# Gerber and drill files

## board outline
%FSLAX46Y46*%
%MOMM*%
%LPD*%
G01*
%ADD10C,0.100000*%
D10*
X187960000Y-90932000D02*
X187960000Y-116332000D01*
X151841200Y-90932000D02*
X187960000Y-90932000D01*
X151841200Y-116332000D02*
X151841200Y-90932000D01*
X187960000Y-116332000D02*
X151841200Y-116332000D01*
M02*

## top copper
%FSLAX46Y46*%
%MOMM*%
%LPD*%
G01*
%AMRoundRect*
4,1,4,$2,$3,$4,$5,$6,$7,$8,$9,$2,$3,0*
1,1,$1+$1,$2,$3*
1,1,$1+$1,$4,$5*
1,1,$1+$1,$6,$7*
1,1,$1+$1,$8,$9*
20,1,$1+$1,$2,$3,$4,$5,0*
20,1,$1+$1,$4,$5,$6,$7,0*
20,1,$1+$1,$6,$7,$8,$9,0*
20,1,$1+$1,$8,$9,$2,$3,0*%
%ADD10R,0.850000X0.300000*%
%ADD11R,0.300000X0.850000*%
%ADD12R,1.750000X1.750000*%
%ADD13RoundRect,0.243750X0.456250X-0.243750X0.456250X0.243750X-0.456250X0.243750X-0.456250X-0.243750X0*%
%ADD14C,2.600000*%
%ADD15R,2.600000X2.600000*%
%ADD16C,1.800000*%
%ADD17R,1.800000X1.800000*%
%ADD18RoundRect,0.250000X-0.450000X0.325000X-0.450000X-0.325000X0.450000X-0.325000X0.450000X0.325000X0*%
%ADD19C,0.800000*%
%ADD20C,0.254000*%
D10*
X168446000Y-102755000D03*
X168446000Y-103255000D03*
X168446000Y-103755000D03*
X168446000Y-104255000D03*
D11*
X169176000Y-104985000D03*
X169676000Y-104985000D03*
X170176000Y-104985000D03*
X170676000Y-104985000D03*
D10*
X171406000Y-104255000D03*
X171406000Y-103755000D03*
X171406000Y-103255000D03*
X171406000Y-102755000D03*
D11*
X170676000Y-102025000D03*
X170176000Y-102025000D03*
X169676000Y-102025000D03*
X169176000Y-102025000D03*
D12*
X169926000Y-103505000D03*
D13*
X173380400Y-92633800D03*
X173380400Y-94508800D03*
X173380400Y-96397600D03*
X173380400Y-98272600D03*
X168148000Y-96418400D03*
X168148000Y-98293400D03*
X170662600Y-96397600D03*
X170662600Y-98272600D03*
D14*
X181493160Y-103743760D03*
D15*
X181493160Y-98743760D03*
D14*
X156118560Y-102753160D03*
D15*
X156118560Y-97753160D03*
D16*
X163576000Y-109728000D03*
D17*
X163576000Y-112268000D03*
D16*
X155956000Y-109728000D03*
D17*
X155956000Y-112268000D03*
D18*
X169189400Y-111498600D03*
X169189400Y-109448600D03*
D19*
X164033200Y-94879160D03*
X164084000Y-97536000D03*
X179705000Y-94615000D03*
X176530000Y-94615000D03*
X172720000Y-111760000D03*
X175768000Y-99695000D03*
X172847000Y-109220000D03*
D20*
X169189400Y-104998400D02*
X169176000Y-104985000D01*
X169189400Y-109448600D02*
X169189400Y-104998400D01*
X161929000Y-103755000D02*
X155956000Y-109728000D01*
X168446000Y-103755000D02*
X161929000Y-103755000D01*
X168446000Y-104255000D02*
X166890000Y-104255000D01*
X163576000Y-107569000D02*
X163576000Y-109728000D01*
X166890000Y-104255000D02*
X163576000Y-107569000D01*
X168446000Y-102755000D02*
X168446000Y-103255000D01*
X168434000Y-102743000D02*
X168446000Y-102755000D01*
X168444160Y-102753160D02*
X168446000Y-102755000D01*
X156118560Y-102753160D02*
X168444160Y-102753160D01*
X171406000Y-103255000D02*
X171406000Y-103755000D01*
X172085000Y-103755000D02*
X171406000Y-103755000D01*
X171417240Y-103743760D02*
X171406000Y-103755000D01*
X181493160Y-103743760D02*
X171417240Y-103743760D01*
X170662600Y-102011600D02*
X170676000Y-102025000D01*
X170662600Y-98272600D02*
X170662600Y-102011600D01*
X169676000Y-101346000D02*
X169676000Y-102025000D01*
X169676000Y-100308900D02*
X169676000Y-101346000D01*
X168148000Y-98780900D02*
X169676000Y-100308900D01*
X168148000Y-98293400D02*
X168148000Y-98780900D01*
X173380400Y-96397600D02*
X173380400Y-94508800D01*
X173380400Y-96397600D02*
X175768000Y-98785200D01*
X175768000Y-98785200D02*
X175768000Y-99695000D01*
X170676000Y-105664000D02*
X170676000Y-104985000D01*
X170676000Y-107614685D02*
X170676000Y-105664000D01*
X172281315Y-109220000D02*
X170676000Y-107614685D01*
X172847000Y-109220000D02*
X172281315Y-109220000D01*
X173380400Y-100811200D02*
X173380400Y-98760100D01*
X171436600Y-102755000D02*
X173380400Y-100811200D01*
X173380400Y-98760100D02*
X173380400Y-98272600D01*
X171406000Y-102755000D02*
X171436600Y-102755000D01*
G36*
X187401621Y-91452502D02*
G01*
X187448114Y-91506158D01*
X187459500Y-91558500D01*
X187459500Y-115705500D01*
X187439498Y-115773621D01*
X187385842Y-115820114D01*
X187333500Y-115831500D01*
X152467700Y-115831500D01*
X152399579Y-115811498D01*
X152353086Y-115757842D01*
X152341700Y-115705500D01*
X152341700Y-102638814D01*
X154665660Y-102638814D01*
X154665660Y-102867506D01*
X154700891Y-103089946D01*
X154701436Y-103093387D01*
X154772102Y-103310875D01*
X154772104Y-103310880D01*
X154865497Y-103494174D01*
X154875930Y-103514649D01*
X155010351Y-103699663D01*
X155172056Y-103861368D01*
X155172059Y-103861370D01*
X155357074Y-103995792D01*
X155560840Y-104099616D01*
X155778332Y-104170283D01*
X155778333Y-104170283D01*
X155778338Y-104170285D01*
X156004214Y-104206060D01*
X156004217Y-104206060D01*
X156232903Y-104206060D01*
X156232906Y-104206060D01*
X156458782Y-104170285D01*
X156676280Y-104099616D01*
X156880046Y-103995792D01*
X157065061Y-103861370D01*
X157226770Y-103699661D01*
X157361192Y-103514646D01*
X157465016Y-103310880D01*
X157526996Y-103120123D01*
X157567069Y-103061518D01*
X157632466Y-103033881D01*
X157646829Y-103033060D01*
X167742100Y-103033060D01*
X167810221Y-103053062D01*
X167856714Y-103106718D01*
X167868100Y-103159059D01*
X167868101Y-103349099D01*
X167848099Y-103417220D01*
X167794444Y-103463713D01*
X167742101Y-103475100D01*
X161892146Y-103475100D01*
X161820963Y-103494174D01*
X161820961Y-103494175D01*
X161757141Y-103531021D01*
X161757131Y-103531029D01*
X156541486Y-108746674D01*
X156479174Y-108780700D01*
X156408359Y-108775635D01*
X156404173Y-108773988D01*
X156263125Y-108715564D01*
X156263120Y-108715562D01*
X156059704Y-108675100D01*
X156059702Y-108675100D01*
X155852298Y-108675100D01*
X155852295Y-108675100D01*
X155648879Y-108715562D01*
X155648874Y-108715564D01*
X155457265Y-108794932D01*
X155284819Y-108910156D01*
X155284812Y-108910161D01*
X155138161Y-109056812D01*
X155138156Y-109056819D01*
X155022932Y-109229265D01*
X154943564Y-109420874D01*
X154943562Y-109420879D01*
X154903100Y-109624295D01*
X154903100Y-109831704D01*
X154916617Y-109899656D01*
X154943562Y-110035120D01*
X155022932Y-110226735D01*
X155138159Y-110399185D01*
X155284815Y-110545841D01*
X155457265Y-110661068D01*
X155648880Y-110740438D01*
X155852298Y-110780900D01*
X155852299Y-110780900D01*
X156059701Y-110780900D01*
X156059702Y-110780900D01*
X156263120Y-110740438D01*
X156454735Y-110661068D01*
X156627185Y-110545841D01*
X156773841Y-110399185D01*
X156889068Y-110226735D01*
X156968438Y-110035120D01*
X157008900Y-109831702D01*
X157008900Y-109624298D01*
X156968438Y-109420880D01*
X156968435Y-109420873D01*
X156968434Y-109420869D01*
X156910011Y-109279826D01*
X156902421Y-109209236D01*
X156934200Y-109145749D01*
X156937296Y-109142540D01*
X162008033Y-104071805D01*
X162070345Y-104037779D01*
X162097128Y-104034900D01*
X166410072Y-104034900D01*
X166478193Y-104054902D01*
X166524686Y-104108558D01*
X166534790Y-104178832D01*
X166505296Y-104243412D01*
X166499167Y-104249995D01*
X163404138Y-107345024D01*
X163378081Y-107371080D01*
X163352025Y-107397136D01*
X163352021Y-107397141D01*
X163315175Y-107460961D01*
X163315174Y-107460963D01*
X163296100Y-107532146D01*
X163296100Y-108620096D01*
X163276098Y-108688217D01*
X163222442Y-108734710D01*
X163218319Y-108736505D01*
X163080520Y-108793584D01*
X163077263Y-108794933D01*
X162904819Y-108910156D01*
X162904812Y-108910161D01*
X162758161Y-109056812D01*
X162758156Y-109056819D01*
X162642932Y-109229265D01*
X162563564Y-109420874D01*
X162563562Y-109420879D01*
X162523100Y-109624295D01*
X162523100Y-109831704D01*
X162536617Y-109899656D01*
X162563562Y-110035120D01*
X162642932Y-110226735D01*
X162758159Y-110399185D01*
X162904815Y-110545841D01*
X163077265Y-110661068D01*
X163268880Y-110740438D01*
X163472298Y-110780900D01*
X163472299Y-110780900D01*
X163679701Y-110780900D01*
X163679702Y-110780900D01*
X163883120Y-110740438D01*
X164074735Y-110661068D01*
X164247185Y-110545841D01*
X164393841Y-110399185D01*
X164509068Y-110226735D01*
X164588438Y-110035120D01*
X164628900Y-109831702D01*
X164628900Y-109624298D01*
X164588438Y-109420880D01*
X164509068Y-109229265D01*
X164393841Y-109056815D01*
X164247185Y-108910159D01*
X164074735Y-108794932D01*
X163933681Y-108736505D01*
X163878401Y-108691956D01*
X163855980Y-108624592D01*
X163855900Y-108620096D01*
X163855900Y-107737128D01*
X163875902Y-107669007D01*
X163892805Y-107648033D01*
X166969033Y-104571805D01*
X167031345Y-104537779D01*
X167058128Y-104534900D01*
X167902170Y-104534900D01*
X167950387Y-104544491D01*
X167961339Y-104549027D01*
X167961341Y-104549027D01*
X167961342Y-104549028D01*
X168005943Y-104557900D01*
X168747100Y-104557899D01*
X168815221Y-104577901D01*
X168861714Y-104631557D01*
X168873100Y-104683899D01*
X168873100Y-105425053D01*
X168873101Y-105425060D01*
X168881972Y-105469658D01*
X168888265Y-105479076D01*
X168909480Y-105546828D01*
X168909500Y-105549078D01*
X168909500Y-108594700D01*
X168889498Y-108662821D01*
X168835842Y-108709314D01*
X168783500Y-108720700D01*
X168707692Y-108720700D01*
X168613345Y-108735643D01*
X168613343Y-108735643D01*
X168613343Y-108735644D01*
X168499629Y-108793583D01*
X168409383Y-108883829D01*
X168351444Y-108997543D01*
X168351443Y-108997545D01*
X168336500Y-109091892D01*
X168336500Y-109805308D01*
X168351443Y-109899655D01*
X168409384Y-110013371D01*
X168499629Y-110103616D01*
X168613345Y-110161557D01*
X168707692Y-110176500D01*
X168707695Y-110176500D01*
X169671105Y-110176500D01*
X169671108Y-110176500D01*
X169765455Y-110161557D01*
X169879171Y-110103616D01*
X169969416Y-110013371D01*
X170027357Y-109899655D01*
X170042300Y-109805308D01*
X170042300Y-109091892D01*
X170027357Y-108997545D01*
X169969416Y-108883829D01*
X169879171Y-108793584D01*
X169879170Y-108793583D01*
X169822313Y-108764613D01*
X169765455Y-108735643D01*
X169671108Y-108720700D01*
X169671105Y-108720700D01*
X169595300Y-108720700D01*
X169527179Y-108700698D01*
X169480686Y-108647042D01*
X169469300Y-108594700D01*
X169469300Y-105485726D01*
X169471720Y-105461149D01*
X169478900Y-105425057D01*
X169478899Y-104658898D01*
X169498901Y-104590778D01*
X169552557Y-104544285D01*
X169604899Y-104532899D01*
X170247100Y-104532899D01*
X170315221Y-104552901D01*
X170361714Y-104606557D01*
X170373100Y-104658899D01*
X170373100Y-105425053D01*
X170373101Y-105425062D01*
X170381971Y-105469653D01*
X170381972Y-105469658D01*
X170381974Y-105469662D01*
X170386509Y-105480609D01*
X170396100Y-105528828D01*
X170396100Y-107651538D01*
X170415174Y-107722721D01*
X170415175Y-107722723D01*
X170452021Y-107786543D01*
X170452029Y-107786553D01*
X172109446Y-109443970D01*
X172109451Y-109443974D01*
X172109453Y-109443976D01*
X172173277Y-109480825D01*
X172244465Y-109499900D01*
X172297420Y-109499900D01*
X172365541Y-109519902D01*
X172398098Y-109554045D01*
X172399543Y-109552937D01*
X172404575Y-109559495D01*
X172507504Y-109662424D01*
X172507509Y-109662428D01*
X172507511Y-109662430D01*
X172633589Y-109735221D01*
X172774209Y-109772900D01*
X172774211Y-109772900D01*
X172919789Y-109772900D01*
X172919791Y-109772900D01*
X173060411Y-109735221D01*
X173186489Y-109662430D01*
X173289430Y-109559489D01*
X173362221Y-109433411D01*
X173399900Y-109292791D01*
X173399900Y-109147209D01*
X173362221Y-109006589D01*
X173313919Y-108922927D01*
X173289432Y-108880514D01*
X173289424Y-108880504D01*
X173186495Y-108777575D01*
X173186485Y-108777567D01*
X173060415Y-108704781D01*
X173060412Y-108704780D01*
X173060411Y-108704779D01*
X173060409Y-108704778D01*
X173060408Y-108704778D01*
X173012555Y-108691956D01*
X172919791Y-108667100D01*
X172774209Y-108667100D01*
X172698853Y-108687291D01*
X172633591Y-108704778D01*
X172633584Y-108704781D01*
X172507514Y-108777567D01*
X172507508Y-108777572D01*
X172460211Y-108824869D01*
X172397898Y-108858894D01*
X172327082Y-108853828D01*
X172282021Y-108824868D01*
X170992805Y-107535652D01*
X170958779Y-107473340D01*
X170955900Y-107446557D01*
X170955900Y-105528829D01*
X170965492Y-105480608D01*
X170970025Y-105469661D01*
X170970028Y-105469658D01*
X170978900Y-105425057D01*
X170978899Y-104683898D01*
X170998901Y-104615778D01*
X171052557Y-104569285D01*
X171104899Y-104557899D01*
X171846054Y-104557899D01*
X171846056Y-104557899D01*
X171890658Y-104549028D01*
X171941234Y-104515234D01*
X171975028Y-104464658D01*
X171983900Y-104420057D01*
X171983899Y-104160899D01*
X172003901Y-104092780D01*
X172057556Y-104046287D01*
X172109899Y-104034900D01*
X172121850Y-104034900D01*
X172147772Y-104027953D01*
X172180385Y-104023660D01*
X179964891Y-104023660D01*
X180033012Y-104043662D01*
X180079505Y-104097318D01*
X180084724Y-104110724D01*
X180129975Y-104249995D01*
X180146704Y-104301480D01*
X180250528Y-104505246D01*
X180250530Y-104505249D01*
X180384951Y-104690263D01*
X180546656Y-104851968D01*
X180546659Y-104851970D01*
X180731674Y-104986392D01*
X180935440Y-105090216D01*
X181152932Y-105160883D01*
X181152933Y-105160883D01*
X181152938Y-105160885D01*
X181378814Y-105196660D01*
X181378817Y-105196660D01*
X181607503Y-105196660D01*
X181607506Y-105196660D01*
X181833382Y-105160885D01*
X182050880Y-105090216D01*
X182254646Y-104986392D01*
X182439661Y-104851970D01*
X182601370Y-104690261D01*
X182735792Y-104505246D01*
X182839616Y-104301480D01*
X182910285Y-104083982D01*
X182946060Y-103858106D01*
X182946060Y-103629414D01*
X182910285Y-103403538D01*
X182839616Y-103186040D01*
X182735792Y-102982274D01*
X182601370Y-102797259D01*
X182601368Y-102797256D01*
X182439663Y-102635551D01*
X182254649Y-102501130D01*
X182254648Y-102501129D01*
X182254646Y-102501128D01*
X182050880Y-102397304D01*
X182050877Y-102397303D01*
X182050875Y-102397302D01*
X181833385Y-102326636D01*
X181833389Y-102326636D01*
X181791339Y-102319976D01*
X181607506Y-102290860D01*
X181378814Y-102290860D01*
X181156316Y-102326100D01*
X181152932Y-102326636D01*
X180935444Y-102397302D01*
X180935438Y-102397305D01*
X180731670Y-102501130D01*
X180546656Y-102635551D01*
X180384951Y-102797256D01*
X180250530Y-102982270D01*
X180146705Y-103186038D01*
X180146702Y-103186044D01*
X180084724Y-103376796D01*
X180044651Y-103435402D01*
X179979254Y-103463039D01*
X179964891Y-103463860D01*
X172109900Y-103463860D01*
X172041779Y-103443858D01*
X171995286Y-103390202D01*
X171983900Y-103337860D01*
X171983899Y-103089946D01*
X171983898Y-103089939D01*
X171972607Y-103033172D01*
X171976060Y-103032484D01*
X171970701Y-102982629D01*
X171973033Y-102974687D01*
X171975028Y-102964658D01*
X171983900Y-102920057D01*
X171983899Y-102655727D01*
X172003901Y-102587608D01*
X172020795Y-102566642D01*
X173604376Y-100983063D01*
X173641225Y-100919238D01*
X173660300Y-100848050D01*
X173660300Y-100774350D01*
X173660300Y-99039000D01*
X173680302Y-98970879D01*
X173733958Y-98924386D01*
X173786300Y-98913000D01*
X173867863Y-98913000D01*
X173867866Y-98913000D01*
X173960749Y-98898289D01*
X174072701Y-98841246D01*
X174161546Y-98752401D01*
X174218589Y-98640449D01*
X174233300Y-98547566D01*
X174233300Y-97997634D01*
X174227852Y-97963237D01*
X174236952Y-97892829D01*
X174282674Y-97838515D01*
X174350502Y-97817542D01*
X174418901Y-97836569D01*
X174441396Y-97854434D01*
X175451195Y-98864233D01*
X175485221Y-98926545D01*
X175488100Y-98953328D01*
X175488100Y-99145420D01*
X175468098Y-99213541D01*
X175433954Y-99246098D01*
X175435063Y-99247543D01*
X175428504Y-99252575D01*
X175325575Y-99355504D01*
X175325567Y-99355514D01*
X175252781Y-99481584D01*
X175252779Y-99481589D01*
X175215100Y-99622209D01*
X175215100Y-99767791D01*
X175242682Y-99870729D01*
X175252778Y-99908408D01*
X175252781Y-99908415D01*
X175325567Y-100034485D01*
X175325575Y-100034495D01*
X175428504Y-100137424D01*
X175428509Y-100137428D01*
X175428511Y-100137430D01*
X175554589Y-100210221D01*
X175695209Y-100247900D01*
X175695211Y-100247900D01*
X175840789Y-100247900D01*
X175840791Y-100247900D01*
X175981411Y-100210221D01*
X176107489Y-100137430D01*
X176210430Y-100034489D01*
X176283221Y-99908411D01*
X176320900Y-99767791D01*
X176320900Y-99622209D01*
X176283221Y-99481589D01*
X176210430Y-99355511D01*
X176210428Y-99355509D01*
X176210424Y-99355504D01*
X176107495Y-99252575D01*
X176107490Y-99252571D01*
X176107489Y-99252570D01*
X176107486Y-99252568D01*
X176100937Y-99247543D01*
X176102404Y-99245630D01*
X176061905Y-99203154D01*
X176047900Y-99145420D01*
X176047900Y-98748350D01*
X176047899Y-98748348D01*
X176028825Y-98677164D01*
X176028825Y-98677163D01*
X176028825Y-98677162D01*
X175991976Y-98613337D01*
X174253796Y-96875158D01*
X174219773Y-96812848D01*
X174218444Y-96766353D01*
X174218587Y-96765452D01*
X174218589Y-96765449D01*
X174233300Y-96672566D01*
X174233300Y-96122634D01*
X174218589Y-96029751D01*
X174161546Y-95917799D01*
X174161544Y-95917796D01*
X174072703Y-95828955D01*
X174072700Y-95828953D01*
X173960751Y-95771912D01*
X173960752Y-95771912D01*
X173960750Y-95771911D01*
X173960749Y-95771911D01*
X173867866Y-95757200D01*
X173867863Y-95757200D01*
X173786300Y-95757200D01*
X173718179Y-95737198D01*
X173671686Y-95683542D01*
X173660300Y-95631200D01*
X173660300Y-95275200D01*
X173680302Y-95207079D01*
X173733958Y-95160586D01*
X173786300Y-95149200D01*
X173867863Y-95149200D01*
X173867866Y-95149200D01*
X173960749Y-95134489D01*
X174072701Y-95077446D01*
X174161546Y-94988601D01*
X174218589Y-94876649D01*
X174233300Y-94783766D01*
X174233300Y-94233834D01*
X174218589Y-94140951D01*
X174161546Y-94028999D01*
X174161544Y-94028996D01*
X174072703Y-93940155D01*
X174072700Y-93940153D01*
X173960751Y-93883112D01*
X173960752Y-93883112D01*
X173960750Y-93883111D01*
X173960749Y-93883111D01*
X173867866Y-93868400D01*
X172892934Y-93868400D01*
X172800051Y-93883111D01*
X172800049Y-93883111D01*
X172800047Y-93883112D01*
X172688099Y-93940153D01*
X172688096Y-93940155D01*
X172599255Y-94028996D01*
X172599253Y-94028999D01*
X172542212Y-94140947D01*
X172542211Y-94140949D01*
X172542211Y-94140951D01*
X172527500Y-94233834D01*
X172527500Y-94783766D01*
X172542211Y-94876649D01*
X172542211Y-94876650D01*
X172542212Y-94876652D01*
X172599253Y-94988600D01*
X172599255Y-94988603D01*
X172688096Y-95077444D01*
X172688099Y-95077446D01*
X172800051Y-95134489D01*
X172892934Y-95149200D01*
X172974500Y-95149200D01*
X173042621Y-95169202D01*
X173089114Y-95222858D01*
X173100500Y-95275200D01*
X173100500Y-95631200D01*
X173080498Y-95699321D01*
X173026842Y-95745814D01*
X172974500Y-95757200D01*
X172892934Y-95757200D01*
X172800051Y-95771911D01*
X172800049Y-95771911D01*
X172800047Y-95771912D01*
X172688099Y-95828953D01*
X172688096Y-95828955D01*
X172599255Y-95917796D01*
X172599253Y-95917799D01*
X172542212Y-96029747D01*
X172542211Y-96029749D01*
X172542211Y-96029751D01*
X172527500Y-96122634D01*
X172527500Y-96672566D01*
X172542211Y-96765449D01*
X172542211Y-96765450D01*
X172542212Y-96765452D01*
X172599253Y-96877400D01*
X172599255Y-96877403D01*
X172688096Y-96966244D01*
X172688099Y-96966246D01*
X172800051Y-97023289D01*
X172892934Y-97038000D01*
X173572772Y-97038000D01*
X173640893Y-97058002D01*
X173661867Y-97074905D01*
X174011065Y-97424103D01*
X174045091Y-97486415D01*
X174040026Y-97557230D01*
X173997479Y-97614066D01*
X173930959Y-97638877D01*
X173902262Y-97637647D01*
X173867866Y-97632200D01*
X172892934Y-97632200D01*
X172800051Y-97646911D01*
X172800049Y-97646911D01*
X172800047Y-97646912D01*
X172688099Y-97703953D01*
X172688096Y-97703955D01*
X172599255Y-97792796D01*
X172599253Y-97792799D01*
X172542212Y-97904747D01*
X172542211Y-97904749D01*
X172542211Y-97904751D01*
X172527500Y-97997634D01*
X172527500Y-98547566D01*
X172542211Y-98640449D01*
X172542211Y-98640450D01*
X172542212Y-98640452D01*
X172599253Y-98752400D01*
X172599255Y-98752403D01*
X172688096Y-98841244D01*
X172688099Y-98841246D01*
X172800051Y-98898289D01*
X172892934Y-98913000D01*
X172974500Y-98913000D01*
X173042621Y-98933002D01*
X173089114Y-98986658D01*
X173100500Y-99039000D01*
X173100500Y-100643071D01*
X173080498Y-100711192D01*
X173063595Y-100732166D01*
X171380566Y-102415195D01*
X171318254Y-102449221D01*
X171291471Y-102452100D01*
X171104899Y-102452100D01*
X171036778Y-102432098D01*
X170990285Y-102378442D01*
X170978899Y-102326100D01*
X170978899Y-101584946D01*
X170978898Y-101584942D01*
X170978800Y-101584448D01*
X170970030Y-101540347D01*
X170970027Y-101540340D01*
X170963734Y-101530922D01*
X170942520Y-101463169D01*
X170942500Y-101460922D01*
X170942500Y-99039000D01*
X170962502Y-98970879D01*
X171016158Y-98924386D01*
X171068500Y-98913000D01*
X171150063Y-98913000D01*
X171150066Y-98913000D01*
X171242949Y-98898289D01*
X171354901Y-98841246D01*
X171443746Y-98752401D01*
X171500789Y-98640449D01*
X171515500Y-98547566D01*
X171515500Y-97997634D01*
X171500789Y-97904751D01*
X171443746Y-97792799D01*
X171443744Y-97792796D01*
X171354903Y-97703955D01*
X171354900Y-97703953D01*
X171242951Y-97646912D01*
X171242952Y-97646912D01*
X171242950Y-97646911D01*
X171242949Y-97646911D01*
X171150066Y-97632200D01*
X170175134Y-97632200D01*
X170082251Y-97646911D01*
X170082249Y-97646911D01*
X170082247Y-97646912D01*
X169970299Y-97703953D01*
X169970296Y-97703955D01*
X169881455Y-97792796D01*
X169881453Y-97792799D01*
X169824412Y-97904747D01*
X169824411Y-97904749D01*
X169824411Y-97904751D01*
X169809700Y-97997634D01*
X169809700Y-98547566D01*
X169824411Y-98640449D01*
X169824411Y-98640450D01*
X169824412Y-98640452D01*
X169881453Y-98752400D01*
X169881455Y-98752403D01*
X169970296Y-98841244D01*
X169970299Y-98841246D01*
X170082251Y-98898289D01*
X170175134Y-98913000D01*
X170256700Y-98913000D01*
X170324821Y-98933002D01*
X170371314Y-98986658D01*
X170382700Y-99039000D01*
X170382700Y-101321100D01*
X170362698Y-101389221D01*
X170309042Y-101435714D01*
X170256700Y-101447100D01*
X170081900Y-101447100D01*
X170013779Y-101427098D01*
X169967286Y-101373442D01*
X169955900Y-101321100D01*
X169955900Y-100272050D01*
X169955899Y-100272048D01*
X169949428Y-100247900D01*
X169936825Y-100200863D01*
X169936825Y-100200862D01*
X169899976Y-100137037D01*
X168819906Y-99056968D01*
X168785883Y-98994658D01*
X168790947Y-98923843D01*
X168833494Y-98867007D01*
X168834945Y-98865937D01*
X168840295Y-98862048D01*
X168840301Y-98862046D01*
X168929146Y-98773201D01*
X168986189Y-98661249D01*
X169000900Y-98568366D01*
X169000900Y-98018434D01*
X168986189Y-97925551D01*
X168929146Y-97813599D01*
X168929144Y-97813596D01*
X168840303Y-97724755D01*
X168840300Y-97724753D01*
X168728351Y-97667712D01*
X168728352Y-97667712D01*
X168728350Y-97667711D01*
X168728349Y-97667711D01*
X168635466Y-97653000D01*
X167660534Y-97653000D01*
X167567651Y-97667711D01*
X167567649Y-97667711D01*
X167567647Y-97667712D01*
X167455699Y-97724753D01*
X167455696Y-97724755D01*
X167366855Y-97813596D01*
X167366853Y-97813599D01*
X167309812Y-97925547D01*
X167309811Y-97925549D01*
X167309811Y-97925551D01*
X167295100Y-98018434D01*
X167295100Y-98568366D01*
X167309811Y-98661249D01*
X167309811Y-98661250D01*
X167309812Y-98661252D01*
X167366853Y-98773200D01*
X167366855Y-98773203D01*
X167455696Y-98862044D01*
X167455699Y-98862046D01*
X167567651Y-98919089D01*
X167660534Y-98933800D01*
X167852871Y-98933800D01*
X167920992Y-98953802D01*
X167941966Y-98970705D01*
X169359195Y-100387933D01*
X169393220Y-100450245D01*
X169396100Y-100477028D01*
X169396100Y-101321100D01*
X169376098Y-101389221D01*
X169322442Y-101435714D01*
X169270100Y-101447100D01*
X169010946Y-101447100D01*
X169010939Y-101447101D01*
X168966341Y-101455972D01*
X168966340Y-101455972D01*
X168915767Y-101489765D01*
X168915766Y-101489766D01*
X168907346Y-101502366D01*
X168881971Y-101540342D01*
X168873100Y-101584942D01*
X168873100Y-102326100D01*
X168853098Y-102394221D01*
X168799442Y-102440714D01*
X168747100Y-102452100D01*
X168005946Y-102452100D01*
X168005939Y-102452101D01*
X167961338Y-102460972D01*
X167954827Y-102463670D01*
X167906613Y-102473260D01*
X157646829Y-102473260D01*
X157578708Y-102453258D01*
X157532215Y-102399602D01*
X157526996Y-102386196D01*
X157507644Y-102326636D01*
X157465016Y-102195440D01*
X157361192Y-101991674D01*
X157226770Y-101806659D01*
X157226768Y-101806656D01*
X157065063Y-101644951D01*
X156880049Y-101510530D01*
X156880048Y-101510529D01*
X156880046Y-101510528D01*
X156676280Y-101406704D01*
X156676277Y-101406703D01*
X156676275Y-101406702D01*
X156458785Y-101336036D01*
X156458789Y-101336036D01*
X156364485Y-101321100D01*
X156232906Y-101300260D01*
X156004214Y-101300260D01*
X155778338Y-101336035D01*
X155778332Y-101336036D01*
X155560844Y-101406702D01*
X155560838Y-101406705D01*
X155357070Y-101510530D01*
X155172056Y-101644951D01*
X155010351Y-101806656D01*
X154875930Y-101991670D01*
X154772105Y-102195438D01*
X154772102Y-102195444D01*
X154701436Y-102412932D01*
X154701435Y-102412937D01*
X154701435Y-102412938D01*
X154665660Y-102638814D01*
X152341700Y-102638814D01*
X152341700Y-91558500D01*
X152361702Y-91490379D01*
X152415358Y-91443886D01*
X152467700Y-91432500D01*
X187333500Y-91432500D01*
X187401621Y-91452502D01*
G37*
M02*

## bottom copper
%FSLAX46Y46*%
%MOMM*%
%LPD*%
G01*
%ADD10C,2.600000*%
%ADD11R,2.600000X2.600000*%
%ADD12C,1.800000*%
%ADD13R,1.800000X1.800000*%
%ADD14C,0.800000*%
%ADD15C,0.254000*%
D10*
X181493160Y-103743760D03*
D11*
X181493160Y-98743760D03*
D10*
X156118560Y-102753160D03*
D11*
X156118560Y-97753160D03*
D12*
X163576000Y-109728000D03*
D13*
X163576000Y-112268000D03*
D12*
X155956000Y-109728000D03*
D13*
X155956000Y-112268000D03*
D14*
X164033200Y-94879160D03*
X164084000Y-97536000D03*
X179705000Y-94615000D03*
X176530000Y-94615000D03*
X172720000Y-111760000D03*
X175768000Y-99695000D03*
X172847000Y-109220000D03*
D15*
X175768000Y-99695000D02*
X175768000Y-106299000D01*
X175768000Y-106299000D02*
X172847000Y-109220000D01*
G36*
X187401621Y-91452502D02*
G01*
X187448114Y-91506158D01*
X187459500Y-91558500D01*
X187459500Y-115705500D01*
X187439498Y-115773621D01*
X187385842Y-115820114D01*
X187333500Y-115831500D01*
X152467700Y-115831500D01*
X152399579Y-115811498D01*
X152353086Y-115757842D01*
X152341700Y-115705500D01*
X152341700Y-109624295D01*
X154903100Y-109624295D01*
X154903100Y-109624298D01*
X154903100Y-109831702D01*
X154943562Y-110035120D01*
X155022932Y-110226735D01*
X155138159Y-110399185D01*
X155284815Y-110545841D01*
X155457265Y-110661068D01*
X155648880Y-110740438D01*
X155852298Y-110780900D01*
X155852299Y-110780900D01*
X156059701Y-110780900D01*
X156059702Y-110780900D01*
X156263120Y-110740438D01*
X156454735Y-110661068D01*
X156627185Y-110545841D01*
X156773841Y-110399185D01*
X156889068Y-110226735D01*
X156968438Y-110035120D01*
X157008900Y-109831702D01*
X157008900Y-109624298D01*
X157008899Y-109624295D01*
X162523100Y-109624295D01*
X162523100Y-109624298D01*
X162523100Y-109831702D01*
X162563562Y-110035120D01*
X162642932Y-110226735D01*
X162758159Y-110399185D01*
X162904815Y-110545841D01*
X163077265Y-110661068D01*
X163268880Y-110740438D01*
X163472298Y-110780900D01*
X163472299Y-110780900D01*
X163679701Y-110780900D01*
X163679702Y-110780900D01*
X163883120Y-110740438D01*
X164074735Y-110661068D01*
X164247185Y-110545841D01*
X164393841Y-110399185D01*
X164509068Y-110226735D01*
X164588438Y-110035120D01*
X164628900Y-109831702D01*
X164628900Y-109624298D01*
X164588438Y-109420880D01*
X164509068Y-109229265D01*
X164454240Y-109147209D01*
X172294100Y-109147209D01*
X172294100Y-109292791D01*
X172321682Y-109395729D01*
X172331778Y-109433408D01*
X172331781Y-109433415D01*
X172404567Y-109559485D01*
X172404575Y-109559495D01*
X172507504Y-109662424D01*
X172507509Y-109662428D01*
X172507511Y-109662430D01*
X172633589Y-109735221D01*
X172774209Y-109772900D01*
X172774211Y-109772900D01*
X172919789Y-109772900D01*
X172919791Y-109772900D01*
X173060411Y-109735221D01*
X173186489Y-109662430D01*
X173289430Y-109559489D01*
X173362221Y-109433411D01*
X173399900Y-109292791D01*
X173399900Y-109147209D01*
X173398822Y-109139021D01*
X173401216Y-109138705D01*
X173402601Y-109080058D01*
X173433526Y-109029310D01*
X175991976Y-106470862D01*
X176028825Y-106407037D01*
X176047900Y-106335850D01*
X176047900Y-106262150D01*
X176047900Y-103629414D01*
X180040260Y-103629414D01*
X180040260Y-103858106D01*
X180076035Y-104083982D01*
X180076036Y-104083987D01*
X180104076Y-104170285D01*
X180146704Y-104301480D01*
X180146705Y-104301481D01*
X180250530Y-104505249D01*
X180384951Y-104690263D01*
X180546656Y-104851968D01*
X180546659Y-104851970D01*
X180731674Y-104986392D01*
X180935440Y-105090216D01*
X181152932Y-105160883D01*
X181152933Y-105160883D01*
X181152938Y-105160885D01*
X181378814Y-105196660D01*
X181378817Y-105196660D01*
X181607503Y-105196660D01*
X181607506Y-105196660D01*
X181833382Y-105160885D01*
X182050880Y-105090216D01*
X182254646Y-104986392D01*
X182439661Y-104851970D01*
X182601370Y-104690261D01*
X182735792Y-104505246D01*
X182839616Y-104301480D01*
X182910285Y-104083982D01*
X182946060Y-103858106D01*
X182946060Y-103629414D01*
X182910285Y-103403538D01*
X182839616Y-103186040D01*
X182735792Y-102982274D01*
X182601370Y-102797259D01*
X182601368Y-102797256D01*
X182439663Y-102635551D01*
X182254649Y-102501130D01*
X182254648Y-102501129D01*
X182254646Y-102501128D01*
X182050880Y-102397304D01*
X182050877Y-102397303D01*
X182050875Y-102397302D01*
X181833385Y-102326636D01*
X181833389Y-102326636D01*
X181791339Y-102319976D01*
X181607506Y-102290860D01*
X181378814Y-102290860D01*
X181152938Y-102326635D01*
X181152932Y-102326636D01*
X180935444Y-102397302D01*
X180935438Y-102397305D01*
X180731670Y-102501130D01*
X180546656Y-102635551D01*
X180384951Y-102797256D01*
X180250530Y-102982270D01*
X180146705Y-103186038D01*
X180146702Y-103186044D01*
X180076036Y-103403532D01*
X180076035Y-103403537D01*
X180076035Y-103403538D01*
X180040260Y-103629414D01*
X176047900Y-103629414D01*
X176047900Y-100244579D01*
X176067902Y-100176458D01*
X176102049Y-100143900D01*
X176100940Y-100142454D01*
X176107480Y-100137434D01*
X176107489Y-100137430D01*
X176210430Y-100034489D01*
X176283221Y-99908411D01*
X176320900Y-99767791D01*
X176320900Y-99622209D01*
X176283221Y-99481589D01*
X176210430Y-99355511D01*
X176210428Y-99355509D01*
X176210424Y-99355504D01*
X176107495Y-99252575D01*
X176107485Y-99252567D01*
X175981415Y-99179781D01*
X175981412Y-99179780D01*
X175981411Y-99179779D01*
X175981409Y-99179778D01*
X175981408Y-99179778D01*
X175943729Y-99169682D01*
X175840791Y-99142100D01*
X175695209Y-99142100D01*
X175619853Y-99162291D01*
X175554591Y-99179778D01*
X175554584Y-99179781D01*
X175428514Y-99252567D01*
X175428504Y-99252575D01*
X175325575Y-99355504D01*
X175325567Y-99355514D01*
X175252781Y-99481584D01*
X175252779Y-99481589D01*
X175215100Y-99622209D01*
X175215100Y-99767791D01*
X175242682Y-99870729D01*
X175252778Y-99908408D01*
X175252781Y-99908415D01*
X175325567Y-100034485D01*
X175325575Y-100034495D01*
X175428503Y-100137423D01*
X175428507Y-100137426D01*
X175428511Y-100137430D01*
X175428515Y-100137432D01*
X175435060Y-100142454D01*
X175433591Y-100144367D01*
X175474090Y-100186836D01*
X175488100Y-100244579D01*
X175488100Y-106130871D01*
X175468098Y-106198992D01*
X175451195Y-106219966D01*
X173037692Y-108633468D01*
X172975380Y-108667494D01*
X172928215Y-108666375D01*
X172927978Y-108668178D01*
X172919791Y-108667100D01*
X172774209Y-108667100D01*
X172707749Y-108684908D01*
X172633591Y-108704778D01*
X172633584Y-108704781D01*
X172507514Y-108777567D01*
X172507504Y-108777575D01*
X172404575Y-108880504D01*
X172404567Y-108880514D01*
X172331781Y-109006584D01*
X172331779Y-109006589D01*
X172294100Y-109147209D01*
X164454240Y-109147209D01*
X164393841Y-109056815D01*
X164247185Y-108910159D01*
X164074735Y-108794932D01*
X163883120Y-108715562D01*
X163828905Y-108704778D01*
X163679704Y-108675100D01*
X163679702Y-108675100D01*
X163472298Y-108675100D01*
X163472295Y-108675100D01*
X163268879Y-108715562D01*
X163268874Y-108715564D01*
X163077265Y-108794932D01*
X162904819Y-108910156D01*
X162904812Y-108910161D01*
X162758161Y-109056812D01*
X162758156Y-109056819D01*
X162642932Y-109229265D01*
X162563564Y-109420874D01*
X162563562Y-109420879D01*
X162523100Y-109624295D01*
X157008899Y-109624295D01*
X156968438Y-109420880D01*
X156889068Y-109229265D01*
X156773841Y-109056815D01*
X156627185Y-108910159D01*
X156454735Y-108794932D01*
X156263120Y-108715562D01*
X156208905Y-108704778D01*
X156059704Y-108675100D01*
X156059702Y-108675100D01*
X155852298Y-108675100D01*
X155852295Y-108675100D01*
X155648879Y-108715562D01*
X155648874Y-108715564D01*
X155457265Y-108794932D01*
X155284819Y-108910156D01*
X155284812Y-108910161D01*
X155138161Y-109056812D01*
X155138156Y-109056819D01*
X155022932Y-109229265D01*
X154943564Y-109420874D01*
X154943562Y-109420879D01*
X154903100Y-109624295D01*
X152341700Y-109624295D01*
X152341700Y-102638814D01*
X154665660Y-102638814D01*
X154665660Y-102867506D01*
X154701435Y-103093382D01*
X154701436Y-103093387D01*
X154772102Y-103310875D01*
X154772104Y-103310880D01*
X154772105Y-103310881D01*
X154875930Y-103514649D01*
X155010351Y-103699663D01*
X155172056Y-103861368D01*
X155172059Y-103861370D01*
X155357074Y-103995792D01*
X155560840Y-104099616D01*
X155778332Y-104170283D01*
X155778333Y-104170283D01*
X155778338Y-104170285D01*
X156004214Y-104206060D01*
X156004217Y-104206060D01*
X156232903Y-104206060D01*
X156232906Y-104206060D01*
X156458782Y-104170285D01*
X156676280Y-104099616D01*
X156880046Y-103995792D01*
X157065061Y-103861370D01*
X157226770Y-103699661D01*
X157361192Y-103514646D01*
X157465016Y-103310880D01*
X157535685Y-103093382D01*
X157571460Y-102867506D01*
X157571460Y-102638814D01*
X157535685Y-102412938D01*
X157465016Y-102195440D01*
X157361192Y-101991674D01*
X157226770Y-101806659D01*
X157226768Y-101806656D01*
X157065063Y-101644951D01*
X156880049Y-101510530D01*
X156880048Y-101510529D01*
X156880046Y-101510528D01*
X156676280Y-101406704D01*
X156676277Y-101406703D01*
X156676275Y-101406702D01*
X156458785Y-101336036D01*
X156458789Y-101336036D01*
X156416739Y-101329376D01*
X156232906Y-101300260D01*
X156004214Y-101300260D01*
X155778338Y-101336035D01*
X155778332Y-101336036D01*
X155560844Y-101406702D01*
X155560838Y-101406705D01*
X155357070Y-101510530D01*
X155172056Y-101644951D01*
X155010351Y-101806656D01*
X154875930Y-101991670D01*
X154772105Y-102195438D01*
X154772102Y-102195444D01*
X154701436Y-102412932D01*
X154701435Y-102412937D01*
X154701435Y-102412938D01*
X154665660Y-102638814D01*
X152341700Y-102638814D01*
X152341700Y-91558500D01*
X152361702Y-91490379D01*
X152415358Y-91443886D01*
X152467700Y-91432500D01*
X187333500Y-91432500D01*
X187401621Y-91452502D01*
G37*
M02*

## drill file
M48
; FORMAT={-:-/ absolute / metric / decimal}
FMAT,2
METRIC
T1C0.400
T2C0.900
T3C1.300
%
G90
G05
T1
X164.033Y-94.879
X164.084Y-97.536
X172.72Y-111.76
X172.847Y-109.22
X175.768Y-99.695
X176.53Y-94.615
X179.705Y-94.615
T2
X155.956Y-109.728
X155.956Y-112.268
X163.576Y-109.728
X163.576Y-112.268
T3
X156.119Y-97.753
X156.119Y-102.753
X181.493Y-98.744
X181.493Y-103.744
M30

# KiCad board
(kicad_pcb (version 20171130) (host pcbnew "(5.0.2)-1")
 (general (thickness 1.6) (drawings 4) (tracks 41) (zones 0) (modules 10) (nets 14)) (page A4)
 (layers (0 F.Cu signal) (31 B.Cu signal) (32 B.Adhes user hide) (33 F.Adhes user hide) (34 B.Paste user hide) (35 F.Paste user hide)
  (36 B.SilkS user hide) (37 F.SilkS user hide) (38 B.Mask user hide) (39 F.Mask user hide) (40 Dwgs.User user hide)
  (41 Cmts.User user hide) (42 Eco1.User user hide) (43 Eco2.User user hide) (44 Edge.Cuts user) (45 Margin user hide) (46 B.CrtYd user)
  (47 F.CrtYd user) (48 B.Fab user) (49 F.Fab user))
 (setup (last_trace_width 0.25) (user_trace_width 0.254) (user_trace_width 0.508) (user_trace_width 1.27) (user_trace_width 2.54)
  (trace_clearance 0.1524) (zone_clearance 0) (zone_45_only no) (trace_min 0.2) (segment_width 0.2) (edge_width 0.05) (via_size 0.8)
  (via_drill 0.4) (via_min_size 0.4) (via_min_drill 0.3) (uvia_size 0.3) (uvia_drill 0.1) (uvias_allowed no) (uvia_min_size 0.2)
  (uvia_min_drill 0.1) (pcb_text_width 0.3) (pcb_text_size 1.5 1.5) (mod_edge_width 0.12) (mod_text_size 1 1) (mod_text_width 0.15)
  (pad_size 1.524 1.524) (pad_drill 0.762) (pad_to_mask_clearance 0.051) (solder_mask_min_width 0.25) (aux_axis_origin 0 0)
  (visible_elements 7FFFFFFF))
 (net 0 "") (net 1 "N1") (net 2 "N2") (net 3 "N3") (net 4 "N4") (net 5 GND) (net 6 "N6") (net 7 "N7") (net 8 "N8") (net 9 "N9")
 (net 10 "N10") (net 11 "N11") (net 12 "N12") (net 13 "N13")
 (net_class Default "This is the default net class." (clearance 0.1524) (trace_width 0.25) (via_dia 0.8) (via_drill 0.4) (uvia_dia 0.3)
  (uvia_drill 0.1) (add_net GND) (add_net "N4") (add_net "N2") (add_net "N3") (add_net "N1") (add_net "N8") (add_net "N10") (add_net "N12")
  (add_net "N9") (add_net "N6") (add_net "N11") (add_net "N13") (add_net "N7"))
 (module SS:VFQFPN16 (layer F.Cu) (at 169.926 103.505)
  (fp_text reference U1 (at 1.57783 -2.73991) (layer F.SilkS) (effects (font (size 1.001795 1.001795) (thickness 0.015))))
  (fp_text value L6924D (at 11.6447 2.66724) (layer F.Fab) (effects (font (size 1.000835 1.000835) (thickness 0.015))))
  (pad 1 smd rect (at -1.48 -0.75) (size 0.85 0.3) (layers F.Cu F.Paste F.Mask) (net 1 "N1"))
  (pad 2 smd rect (at -1.48 -0.25) (size 0.85 0.3) (layers F.Cu F.Paste F.Mask) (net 1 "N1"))
  (pad 3 smd rect (at -1.48 0.25) (size 0.85 0.3) (layers F.Cu F.Paste F.Mask) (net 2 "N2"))
  (pad 4 smd rect (at -1.48 0.75) (size 0.85 0.3) (layers F.Cu F.Paste F.Mask) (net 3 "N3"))
  (pad 5 smd rect (at -0.75 1.48) (size 0.3 0.85) (layers F.Cu F.Paste F.Mask) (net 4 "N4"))
  (pad 6 smd rect (at -0.25 1.48) (size 0.3 0.85) (layers F.Cu F.Paste F.Mask) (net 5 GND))
  (pad 7 smd rect (at 0.25 1.48) (size 0.3 0.85) (layers F.Cu F.Paste F.Mask) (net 5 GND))
  (pad 8 smd rect (at 0.75 1.48) (size 0.3 0.85) (layers F.Cu F.Paste F.Mask) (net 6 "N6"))
  (pad 9 smd rect (at 1.48 0.75) (size 0.85 0.3) (layers F.Cu F.Paste F.Mask) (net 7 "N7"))
  (pad 10 smd rect (at 1.48 0.25) (size 0.85 0.3) (layers F.Cu F.Paste F.Mask) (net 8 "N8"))
  (pad 11 smd rect (at 1.48 -0.25) (size 0.85 0.3) (layers F.Cu F.Paste F.Mask) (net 8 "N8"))
  (pad 12 smd rect (at 1.48 -0.75) (size 0.85 0.3) (layers F.Cu F.Paste F.Mask) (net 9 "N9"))
  (pad 13 smd rect (at 0.75 -1.48) (size 0.3 0.85) (layers F.Cu F.Paste F.Mask) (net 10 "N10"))
  (pad 14 smd rect (at 0.25 -1.48) (size 0.3 0.85) (layers F.Cu F.Paste F.Mask) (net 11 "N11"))
  (pad 15 smd rect (at -0.25 -1.48) (size 0.3 0.85) (layers F.Cu F.Paste F.Mask) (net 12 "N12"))
  (pad 16 smd rect (at -0.75 -1.48) (size 0.3 0.85) (layers F.Cu F.Paste F.Mask) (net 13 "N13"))
  (pad 17 smd rect (at 0 0) (size 1.75 1.75) (layers F.Cu F.Paste F.Mask)))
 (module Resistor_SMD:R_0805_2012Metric (layer F.Cu) (at 173.3804 93.5713 90)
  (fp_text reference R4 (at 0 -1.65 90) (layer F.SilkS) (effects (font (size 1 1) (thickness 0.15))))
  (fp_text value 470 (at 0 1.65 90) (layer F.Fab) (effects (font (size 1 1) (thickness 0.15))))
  (pad 2 smd roundrect (at 0.9375 0 90) (size 0.975 1.4) (layers F.Cu F.Paste F.Mask) (roundrect_rratio 0.25) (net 5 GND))
  (pad 1 smd roundrect (at -0.9375 0 90) (size 0.975 1.4) (layers F.Cu F.Paste F.Mask) (roundrect_rratio 0.25) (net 6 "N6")))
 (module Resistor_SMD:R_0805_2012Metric (layer F.Cu) (at 173.3804 97.3351 90)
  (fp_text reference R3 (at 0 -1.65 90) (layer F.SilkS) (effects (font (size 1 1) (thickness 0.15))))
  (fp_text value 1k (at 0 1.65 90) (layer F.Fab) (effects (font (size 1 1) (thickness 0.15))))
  (pad 2 smd roundrect (at 0.9375 0 90) (size 0.975 1.4) (layers F.Cu F.Paste F.Mask) (roundrect_rratio 0.25) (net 6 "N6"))
  (pad 1 smd roundrect (at -0.9375 0 90) (size 0.975 1.4) (layers F.Cu F.Paste F.Mask) (roundrect_rratio 0.25) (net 9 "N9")))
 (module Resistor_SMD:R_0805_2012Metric (layer F.Cu) (at 168.148 97.3559 90)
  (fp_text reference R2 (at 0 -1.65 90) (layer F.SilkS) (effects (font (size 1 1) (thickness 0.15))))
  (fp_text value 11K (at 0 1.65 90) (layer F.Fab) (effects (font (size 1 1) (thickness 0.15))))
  (pad 2 smd roundrect (at 0.9375 0 90) (size 0.975 1.4) (layers F.Cu F.Paste F.Mask) (roundrect_rratio 0.25) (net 5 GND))
  (pad 1 smd roundrect (at -0.9375 0 90) (size 0.975 1.4) (layers F.Cu F.Paste F.Mask) (roundrect_rratio 0.25) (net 12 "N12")))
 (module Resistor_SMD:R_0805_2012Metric (layer F.Cu) (at 170.6626 97.3351 90)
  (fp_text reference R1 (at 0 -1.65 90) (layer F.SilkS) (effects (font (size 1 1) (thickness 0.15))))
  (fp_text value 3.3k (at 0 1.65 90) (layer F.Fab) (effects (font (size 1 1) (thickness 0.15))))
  (pad 2 smd roundrect (at 0.9375 0 90) (size 0.975 1.4) (layers F.Cu F.Paste F.Mask) (roundrect_rratio 0.25) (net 5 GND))
  (pad 1 smd roundrect (at -0.9375 0 90) (size 0.975 1.4) (layers F.Cu F.Paste F.Mask) (roundrect_rratio 0.25) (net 10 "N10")))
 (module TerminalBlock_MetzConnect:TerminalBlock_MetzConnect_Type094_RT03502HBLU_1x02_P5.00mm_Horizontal (layer F.Cu)
  (at 181.49316 98.74376 270)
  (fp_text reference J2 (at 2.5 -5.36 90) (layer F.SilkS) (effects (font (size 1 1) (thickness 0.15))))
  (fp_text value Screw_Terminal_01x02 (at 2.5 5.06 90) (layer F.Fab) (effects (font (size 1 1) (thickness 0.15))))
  (pad 2 thru_hole circle (at 5 0 270) (size 2.6 2.6) (drill 1.3) (layers *.Cu *.Mask) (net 8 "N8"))
  (pad 1 thru_hole rect (at 0 0 270) (size 2.6 2.6) (drill 1.3) (layers *.Cu *.Mask) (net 5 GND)))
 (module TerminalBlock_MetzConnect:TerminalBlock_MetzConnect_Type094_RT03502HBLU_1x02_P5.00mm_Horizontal (layer F.Cu)
  (at 156.11856 97.75316 270)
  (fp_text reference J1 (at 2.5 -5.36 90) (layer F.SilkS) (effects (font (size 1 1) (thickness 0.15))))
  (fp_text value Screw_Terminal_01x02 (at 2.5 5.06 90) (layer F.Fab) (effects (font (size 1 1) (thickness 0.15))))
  (pad 2 thru_hole circle (at 5 0 270) (size 2.6 2.6) (drill 1.3) (layers *.Cu *.Mask) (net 1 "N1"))
  (pad 1 thru_hole rect (at 0 0 270) (size 2.6 2.6) (drill 1.3) (layers *.Cu *.Mask) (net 5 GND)))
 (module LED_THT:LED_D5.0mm (layer F.Cu) (at 163.576 112.268 90)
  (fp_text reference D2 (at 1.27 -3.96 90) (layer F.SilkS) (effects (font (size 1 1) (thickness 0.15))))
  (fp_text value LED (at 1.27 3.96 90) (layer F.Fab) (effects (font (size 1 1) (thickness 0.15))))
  (pad 2 thru_hole circle (at 2.54 0 90) (size 1.8 1.8) (drill 0.9) (layers *.Cu *.Mask) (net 3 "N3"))
  (pad 1 thru_hole rect (at 0 0 90) (size 1.8 1.8) (drill 0.9) (layers *.Cu *.Mask) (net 5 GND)))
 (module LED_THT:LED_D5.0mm (layer F.Cu) (at 155.956 112.268 90)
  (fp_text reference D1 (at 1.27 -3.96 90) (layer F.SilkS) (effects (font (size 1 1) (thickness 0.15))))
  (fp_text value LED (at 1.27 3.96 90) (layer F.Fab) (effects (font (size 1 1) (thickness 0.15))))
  (pad 2 thru_hole circle (at 2.54 0 90) (size 1.8 1.8) (drill 0.9) (layers *.Cu *.Mask) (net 2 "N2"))
  (pad 1 thru_hole rect (at 0 0 90) (size 1.8 1.8) (drill 0.9) (layers *.Cu *.Mask) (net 5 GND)))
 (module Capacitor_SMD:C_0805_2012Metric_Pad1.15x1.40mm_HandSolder (layer F.Cu) (at 169.1894 110.4736 270)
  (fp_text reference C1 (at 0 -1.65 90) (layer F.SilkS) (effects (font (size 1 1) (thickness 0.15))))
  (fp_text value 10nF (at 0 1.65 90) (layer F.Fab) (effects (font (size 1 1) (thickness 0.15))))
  (pad 2 smd roundrect (at 1.025 0 270) (size 1.15 1.4) (layers F.Cu F.Paste F.Mask) (roundrect_rratio 0.217391) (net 5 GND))
  (pad 1 smd roundrect (at -1.025 0 270) (size 1.15 1.4) (layers F.Cu F.Paste F.Mask) (roundrect_rratio 0.217391) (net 4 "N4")))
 (gr_line (start 187.96 90.932) (end 187.96 116.332) (layer Edge.Cuts) (width 0.1))
 (gr_line (start 151.8412 90.932) (end 187.96 90.932) (layer Edge.Cuts) (width 0.1))
 (gr_line (start 151.8412 116.332) (end 151.8412 90.932) (layer Edge.Cuts) (width 0.1))
 (gr_line (start 187.96 116.332) (end 151.8412 116.332) (layer Edge.Cuts) (width 0.1))
 (via (at 164.0332 94.87916) (size 0.8) (drill 0.4) (layers F.Cu B.Cu) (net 5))
 (via (at 164.084 97.536) (size 0.8) (drill 0.4) (layers F.Cu B.Cu) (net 5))
 (via (at 179.705 94.615) (size 0.8) (drill 0.4) (layers F.Cu B.Cu) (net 5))
 (via (at 176.53 94.615) (size 0.8) (drill 0.4) (layers F.Cu B.Cu) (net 5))
 (via (at 172.72 111.76) (size 0.8) (drill 0.4) (layers F.Cu B.Cu) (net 5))
 (segment (start 169.1894 104.9984) (end 169.176 104.985) (width 0.254) (layer F.Cu) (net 4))
 (segment (start 169.1894 109.4486) (end 169.1894 104.9984) (width 0.254) (layer F.Cu) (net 4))
 (segment (start 161.929 103.755) (end 155.956 109.728) (width 0.254) (layer F.Cu) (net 2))
 (segment (start 168.446 103.755) (end 161.929 103.755) (width 0.254) (layer F.Cu) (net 2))
 (segment (start 168.446 104.255) (end 166.89 104.255) (width 0.254) (layer F.Cu) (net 3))
 (segment (start 163.576 107.569) (end 163.576 109.728) (width 0.254) (layer F.Cu) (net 3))
 (segment (start 166.89 104.255) (end 163.576 107.569) (width 0.254) (layer F.Cu) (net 3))
 (segment (start 168.446 102.755) (end 168.446 103.255) (width 0.254) (layer F.Cu) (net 1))
 (segment (start 168.434 102.743) (end 168.446 102.755) (width 0.254) (layer F.Cu) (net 1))
 (segment (start 168.44416 102.75316) (end 168.446 102.755) (width 0.254) (layer F.Cu) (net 1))
 (segment (start 156.11856 102.75316) (end 168.44416 102.75316) (width 0.254) (layer F.Cu) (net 1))
 (segment (start 171.406 103.255) (end 171.406 103.755) (width 0.254) (layer F.Cu) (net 8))
 (segment (start 172.085 103.755) (end 171.406 103.755) (width 0.254) (layer F.Cu) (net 8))
 (segment (start 171.41724 103.74376) (end 171.406 103.755) (width 0.254) (layer F.Cu) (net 8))
 (segment (start 181.49316 103.74376) (end 171.41724 103.74376) (width 0.254) (layer F.Cu) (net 8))
 (segment (start 170.6626 102.0116) (end 170.676 102.025) (width 0.254) (layer F.Cu) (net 10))
 (segment (start 170.6626 98.2726) (end 170.6626 102.0116) (width 0.254) (layer F.Cu) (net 10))
 (segment (start 169.676 101.346) (end 169.676 102.025) (width 0.254) (layer F.Cu) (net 12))
 (segment (start 169.676 100.3089) (end 169.676 101.346) (width 0.254) (layer F.Cu) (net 12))
 (segment (start 168.148 98.7809) (end 169.676 100.3089) (width 0.254) (layer F.Cu) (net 12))
 (segment (start 168.148 98.2934) (end 168.148 98.7809) (width 0.254) (layer F.Cu) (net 12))
 (segment (start 173.3804 96.3976) (end 173.3804 94.5088) (width 0.254) (layer F.Cu) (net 6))
 (segment (start 173.3804 96.3976) (end 175.768 98.7852) (width 0.254) (layer F.Cu) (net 6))
 (via (at 175.768 99.695) (size 0.8) (drill 0.4) (layers F.Cu B.Cu) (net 6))
 (segment (start 175.768 98.7852) (end 175.768 99.695) (width 0.254) (layer F.Cu) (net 6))
 (segment (start 175.768 99.695) (end 175.768 106.299) (width 0.254) (layer B.Cu) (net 6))
 (segment (start 175.768 106.299) (end 172.847 109.22) (width 0.254) (layer B.Cu) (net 6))
 (via (at 172.847 109.22) (size 0.8) (drill 0.4) (layers F.Cu B.Cu) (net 6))
 (segment (start 170.676 105.664) (end 170.676 104.985) (width 0.254) (layer F.Cu) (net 6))
 (segment (start 170.676 107.614685) (end 170.676 105.664) (width 0.254) (layer F.Cu) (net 6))
 (segment (start 172.281315 109.22) (end 170.676 107.614685) (width 0.254) (layer F.Cu) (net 6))
 (segment (start 172.847 109.22) (end 172.281315 109.22) (width 0.254) (layer F.Cu) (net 6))
 (segment (start 173.3804 100.8112) (end 173.3804 98.7601) (width 0.254) (layer F.Cu) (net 9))
 (segment (start 171.4366 102.755) (end 173.3804 100.8112) (width 0.254) (layer F.Cu) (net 9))
 (segment (start 173.3804 98.7601) (end 173.3804 98.2726) (width 0.254) (layer F.Cu) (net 9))
 (segment (start 171.406 102.755) (end 171.4366 102.755) (width 0.254) (layer F.Cu) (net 9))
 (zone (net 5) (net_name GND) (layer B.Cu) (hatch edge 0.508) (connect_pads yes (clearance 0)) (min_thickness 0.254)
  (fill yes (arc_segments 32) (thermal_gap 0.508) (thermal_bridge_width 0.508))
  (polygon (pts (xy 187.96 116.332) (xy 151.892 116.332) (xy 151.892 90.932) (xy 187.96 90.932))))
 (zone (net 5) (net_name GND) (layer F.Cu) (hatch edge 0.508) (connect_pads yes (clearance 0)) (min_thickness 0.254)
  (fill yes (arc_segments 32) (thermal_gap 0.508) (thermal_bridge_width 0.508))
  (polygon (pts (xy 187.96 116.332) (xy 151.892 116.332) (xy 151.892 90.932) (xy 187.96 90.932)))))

